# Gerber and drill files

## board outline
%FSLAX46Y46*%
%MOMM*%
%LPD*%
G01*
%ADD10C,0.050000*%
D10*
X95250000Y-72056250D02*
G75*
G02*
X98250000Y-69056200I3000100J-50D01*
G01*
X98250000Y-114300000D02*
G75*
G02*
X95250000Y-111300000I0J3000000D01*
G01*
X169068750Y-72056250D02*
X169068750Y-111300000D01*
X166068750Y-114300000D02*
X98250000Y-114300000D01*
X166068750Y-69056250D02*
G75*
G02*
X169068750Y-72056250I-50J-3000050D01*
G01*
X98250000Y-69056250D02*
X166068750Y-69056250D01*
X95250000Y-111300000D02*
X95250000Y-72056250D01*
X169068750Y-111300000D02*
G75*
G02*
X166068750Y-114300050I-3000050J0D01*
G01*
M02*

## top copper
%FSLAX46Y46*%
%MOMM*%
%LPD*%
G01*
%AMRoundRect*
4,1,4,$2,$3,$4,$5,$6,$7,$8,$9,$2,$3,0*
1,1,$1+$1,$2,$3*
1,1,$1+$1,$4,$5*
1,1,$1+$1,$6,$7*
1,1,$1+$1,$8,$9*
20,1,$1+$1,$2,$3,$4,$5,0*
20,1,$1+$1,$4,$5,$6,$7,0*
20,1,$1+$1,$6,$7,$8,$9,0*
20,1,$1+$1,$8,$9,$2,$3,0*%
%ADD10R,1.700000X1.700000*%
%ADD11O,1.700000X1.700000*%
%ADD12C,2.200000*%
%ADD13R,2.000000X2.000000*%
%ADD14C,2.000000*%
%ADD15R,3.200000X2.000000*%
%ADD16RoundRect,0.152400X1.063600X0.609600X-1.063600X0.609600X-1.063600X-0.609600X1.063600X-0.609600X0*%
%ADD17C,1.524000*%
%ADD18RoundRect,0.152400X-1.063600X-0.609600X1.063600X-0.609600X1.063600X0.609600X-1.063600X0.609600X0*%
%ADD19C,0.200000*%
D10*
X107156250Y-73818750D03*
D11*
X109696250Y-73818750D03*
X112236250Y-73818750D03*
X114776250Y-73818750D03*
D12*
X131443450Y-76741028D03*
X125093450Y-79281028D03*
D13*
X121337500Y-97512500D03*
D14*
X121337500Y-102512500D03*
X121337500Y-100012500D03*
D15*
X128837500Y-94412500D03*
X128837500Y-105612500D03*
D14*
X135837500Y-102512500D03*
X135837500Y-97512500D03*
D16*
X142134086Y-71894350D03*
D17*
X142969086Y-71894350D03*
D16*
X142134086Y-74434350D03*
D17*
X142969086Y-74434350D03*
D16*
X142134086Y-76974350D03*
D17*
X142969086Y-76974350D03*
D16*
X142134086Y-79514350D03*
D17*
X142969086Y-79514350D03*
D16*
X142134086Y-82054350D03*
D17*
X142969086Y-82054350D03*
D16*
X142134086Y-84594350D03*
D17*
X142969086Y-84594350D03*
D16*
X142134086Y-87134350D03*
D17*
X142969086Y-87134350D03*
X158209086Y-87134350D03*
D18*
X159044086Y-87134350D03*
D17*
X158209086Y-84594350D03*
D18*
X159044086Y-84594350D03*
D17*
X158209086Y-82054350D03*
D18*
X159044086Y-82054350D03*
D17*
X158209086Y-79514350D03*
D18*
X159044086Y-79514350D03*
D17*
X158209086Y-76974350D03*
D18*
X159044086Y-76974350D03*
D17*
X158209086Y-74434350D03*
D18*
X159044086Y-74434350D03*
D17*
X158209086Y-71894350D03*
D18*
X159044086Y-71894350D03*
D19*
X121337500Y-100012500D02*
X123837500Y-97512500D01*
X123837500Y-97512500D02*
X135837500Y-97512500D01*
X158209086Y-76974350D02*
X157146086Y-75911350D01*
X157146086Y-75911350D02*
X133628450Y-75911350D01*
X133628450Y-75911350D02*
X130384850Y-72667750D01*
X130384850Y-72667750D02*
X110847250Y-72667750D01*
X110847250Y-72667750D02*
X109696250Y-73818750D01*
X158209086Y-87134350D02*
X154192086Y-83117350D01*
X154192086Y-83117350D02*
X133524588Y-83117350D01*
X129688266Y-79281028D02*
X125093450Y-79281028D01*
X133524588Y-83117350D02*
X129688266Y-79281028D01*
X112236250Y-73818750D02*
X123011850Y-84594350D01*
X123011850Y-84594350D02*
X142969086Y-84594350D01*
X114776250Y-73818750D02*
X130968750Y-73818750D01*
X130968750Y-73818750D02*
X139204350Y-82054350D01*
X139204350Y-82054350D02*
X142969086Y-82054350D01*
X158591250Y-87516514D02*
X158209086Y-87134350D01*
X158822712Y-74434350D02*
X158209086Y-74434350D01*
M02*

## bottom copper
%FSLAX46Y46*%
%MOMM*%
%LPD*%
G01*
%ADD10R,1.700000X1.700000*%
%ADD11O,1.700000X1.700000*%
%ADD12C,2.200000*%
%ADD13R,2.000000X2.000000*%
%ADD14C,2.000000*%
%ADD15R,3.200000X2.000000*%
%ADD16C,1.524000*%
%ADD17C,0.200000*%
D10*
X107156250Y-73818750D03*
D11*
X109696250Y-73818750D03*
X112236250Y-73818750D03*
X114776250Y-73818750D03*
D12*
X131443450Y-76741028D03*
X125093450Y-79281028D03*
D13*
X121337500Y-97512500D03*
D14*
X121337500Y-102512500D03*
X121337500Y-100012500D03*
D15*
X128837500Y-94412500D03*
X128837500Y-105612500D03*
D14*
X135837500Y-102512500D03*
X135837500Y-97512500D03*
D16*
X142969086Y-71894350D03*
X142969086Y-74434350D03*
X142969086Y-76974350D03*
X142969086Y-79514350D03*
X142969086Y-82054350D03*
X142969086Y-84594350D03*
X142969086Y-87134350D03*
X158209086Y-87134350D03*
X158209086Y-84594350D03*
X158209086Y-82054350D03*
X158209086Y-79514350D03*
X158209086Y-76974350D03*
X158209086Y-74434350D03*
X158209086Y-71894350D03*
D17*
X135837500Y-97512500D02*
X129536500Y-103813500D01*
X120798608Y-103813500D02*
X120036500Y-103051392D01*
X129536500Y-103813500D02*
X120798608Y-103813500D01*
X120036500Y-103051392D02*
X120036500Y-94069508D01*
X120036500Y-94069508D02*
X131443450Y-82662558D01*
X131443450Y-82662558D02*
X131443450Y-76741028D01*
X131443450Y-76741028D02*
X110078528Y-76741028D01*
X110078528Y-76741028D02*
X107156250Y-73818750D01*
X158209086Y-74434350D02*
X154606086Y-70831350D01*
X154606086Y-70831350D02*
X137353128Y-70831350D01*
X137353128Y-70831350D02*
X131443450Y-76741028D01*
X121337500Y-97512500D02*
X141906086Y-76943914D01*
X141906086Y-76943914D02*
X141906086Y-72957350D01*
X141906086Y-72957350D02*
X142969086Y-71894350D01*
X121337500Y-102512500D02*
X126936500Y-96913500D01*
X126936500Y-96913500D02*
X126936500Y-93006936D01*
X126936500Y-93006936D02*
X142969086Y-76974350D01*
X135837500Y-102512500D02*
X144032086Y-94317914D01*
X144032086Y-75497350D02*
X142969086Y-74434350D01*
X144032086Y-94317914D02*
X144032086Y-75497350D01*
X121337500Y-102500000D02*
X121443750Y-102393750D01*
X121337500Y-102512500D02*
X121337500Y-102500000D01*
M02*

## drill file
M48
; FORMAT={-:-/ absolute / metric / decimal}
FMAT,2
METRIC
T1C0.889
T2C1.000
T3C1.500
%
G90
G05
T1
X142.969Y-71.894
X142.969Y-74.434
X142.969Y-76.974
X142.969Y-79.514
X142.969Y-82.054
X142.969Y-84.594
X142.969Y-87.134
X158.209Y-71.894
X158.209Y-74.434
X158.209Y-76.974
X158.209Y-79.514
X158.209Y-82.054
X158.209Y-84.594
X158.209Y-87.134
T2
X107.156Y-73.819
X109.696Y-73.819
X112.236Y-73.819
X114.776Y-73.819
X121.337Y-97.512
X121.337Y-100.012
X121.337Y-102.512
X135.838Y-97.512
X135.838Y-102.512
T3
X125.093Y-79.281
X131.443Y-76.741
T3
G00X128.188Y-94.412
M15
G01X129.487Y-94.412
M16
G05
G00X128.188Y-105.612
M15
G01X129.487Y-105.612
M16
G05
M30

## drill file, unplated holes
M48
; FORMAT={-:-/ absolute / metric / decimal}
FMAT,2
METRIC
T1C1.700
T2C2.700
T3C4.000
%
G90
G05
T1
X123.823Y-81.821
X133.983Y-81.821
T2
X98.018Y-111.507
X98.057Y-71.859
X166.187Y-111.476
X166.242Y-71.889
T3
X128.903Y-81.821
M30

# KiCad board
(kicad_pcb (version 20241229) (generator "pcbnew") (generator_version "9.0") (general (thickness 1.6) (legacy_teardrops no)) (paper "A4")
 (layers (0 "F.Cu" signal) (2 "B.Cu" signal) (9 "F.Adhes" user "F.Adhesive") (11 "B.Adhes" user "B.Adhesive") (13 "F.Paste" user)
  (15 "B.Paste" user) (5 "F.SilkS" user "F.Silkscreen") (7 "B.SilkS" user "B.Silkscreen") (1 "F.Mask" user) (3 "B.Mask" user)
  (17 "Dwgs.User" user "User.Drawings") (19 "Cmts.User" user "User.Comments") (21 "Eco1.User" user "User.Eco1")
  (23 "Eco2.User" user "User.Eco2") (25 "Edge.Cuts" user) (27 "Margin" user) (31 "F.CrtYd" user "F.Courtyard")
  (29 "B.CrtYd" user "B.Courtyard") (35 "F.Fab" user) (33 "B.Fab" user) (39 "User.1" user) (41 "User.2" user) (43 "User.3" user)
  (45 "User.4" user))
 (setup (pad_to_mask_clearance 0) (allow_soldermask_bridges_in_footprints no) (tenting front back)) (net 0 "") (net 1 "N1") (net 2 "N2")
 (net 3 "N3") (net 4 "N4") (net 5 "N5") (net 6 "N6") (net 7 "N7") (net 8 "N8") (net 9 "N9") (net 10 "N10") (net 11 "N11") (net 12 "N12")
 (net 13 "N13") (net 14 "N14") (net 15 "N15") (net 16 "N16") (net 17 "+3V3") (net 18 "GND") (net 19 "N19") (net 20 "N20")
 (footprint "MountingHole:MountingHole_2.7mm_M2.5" (layer "F.Cu") (at 166.241551 71.889468)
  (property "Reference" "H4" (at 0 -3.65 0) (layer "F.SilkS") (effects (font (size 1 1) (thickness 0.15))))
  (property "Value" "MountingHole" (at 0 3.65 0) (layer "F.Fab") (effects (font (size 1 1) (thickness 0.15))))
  (pad "" np_thru_hole circle (at 0 0) (size 2.7 2.7) (drill 2.7) (layers "*.Cu" "*.Mask")))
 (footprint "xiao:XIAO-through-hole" (layer "F.Cu") (at 150.589086 79.51435)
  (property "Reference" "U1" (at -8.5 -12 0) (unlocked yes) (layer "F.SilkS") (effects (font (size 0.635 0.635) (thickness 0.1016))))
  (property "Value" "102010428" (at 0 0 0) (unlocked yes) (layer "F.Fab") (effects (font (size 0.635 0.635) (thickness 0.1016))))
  (pad "1" smd roundrect (at -8.455 -7.62 180) (size 2.432 1.524) (layers "F.Cu" "F.Mask") (roundrect_rratio 0.1) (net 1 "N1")
   (thermal_bridge_angle 45))
  (pad "1" thru_hole circle (at -7.62 -7.62 180) (size 1.524 1.524) (drill 0.889) (layers "*.Cu" "*.Mask") (remove_unused_layers no)
   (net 1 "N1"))
  (pad "2" smd roundrect (at -8.455 -5.08 180) (size 2.432 1.524) (layers "F.Cu" "F.Mask") (roundrect_rratio 0.1) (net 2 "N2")
   (thermal_bridge_angle 45))
  (pad "2" thru_hole circle (at -7.62 -5.08 180) (size 1.524 1.524) (drill 0.889) (layers "*.Cu" "*.Mask") (remove_unused_layers no)
   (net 2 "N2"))
  (pad "3" smd roundrect (at -8.455 -2.54 180) (size 2.432 1.524) (layers "F.Cu" "F.Mask") (roundrect_rratio 0.1) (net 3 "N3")
   (thermal_bridge_angle 45))
  (pad "3" thru_hole circle (at -7.62 -2.54 180) (size 1.524 1.524) (drill 0.889) (layers "*.Cu" "*.Mask") (remove_unused_layers no)
   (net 3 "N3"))
  (pad "4" smd roundrect (at -8.455 0 180) (size 2.432 1.524) (layers "F.Cu" "F.Mask") (roundrect_rratio 0.1) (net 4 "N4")
   (thermal_bridge_angle 45))
  (pad "4" thru_hole circle (at -7.62 0 180) (size 1.524 1.524) (drill 0.889) (layers "*.Cu" "*.Mask") (remove_unused_layers no)
   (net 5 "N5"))
  (pad "5" smd roundrect (at -8.455 2.54 180) (size 2.432 1.524) (layers "F.Cu" "F.Mask") (roundrect_rratio 0.1) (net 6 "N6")
   (thermal_bridge_angle 45))
  (pad "5" thru_hole circle (at -7.62 2.54 180) (size 1.524 1.524) (drill 0.889) (layers "*.Cu" "*.Mask") (remove_unused_layers no)
   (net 6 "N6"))
  (pad "6" smd roundrect (at -8.455 5.08 180) (size 2.432 1.524) (layers "F.Cu" "F.Mask") (roundrect_rratio 0.1) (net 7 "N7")
   (thermal_bridge_angle 45))
  (pad "6" thru_hole circle (at -7.62 5.08 180) (size 1.524 1.524) (drill 0.889) (layers "*.Cu" "*.Mask") (remove_unused_layers no)
   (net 7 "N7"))
  (pad "7" smd roundrect (at -8.455 7.62 180) (size 2.432 1.524) (layers "F.Cu" "F.Mask") (roundrect_rratio 0.1) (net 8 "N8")
   (thermal_bridge_angle 45))
  (pad "7" thru_hole circle (at -7.62 7.62 180) (size 1.524 1.524) (drill 0.889) (layers "*.Cu" "*.Mask") (remove_unused_layers no)
   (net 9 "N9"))
  (pad "8" thru_hole circle (at 7.62 7.62) (size 1.524 1.524) (drill 0.889) (layers "*.Cu" "*.Mask") (remove_unused_layers no)
   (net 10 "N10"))
  (pad "8" smd roundrect (at 8.455 7.62) (size 2.432 1.524) (layers "F.Cu" "F.Mask") (roundrect_rratio 0.1) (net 10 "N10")
   (thermal_bridge_angle 45))
  (pad "9" thru_hole circle (at 7.62 5.08) (size 1.524 1.524) (drill 0.889) (layers "*.Cu" "*.Mask") (remove_unused_layers no)
   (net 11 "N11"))
  (pad "9" smd roundrect (at 8.455 5.08) (size 2.432 1.524) (layers "F.Cu" "F.Mask") (roundrect_rratio 0.1) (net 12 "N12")
   (thermal_bridge_angle 45))
  (pad "10" thru_hole circle (at 7.62 2.54) (size 1.524 1.524) (drill 0.889) (layers "*.Cu" "*.Mask") (remove_unused_layers no)
   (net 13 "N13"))
  (pad "10" smd roundrect (at 8.455 2.54) (size 2.432 1.524) (layers "F.Cu" "F.Mask") (roundrect_rratio 0.1) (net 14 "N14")
   (thermal_bridge_angle 45))
  (pad "11" thru_hole circle (at 7.62 0) (size 1.524 1.524) (drill 0.889) (layers "*.Cu" "*.Mask") (remove_unused_layers no) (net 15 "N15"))
  (pad "11" smd roundrect (at 8.455 0) (size 2.432 1.524) (layers "F.Cu" "F.Mask") (roundrect_rratio 0.1) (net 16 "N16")
   (thermal_bridge_angle 45))
  (pad "12" thru_hole circle (at 7.62 -2.54) (size 1.524 1.524) (drill 0.889) (layers "*.Cu" "*.Mask") (remove_unused_layers no)
   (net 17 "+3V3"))
  (pad "12" smd roundrect (at 8.455 -2.54) (size 2.432 1.524) (layers "F.Cu" "F.Mask") (roundrect_rratio 0.1) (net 17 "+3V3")
   (thermal_bridge_angle 45))
  (pad "13" thru_hole circle (at 7.62 -5.08) (size 1.524 1.524) (drill 0.889) (layers "*.Cu" "*.Mask") (remove_unused_layers no)
   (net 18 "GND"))
  (pad "13" smd roundrect (at 8.455 -5.08) (size 2.432 1.524) (layers "F.Cu" "F.Mask") (roundrect_rratio 0.1) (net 18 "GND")
   (thermal_bridge_angle 45))
  (pad "14" thru_hole circle (at 7.62 -7.62) (size 1.524 1.524) (drill 0.889) (layers "*.Cu" "*.Mask") (remove_unused_layers no)
   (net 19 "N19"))
  (pad "14" smd roundrect (at 8.455 -7.62) (size 2.432 1.524) (layers "F.Cu" "F.Mask") (roundrect_rratio 0.1) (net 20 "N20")
   (thermal_bridge_angle 45)))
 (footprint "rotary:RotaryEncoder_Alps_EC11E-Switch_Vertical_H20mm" (layer "F.Cu") (at 121.3375 97.5125)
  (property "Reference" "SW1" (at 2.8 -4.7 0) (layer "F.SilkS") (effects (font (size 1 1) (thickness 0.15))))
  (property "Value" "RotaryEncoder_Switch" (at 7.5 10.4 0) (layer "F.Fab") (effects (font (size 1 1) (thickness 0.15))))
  (pad "A" thru_hole rect (at 0 0) (size 2 2) (drill 1) (layers "*.Cu" "*.Mask") (remove_unused_layers no) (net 1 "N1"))
  (pad "B" thru_hole circle (at 0 5) (size 2 2) (drill 1) (layers "*.Cu" "*.Mask") (remove_unused_layers no) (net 3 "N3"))
  (pad "C" thru_hole circle (at 0 2.5) (size 2 2) (drill 1) (layers "*.Cu" "*.Mask") (remove_unused_layers no) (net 18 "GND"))
  (pad "MP" thru_hole rect (at 7.5 -3.1) (size 3.2 2) (drill oval 2.8 1.5) (layers "*.Cu" "*.Mask") (remove_unused_layers no))
  (pad "MP" thru_hole rect (at 7.5 8.1) (size 3.2 2) (drill oval 2.8 1.5) (layers "*.Cu" "*.Mask") (remove_unused_layers no))
  (pad "S1" thru_hole circle (at 14.5 5) (size 2 2) (drill 1) (layers "*.Cu" "*.Mask") (remove_unused_layers no) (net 2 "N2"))
  (pad "S2" thru_hole circle (at 14.5 0) (size 2 2) (drill 1) (layers "*.Cu" "*.Mask") (remove_unused_layers no) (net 18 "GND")))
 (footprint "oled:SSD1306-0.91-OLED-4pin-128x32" (layer "F.Cu") (at 104.96625 110.31875 90)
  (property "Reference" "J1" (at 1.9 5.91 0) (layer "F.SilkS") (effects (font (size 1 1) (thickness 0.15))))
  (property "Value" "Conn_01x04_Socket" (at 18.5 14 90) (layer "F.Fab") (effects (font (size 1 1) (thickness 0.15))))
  (pad "1" thru_hole rect (at 36.5 2.19 90) (size 1.7 1.7) (drill 1) (layers "*.Cu" "*.Mask") (remove_unused_layers no) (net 18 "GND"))
  (pad "2" thru_hole oval (at 36.5 4.73 90) (size 1.7 1.7) (drill 1) (layers "*.Cu" "*.Mask") (remove_unused_layers no) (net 17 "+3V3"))
  (pad "3" thru_hole oval (at 36.5 7.27 90) (size 1.7 1.7) (drill 1) (layers "*.Cu" "*.Mask") (remove_unused_layers no) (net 7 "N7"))
  (pad "4" thru_hole oval (at 36.5 9.81 90) (size 1.7 1.7) (drill 1) (layers "*.Cu" "*.Mask") (remove_unused_layers no) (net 6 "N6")))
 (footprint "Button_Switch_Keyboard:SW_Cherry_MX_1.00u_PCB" (layer "F.Cu") (at 131.44345 76.741028)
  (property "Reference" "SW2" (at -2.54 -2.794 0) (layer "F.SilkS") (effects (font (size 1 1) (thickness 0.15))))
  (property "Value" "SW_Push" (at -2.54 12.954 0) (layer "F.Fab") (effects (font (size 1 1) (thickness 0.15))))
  (pad "" np_thru_hole circle (at -7.62 5.08) (size 1.7 1.7) (drill 1.7) (layers "*.Cu" "*.Mask"))
  (pad "" np_thru_hole circle (at -2.54 5.08) (size 4 4) (drill 4) (layers "*.Cu" "*.Mask"))
  (pad "" np_thru_hole circle (at 2.54 5.08) (size 1.7 1.7) (drill 1.7) (layers "*.Cu" "*.Mask"))
  (pad "1" thru_hole circle (at 0 0) (size 2.2 2.2) (drill 1.5) (layers "*.Cu" "*.Mask") (remove_unused_layers no) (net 18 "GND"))
  (pad "2" thru_hole circle (at -6.35 2.54) (size 2.2 2.2) (drill 1.5) (layers "*.Cu" "*.Mask") (remove_unused_layers no) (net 10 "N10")))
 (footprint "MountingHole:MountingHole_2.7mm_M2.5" (layer "F.Cu") (at 98.056834 71.858552)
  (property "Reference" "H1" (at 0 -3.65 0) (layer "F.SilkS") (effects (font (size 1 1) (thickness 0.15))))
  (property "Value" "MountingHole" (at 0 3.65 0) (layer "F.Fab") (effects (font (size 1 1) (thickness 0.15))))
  (pad "" np_thru_hole circle (at 0 0) (size 2.7 2.7) (drill 2.7) (layers "*.Cu" "*.Mask")))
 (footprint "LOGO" (layer "F.Cu") (at 147.6375 100.0125)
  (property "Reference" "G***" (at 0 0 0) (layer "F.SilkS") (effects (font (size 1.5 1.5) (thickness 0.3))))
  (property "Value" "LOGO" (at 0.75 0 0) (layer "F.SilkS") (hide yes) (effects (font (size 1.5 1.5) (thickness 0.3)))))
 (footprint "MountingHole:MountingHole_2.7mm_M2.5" (layer "F.Cu") (at 166.186859 111.475774)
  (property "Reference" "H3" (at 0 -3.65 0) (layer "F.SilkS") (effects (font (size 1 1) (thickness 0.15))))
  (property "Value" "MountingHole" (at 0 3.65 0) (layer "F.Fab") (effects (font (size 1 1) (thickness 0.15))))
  (pad "" np_thru_hole circle (at 0 0) (size 2.7 2.7) (drill 2.7) (layers "*.Cu" "*.Mask")))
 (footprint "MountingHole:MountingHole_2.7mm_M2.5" (layer "F.Cu") (at 98.017649 111.507208)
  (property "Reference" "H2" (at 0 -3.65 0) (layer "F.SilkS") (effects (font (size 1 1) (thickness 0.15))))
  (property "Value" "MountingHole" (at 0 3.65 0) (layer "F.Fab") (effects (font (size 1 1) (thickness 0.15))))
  (pad "" np_thru_hole circle (at 0 0) (size 2.7 2.7) (drill 2.7) (layers "*.Cu" "*.Mask")))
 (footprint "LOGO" (layer "B.Cu") (at 130.96875 90.4875 180)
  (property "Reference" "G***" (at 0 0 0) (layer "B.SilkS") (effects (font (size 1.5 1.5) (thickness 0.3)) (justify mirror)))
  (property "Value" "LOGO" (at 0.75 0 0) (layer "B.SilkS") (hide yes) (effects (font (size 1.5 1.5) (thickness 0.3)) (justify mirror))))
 (gr_arc (start 95.25 72.05625) (mid 96.128697 69.934962) (end 98.25 69.05625) (stroke (width 0.05) (type default)) (layer "Edge.Cuts"))
 (gr_arc (start 98.25 114.3) (mid 96.12868 113.42132) (end 95.25 111.3) (stroke (width 0.05) (type default)) (layer "Edge.Cuts"))
 (gr_line (start 169.06875 72.05625) (end 169.06875 111.3) (stroke (width 0.05) (type default)) (layer "Edge.Cuts"))
 (gr_line (start 166.06875 114.3) (end 98.25 114.3) (stroke (width 0.05) (type default)) (layer "Edge.Cuts"))
 (gr_arc (start 166.06875 69.05625) (mid 168.19007 69.93493) (end 169.06875 72.05625) (stroke (width 0.05) (type default))
  (layer "Edge.Cuts"))
 (gr_line (start 98.25 69.05625) (end 166.06875 69.05625) (stroke (width 0.05) (type default)) (layer "Edge.Cuts"))
 (gr_line (start 95.25 111.3) (end 95.25 72.05625) (stroke (width 0.05) (type default)) (layer "Edge.Cuts"))
 (gr_arc (start 169.06875 111.3) (mid 168.19007 113.42132) (end 166.06875 114.3) (stroke (width 0.05) (type default)) (layer "Edge.Cuts"))
 (segment (start 158.209086 76.97435) (end 157.146086 75.91135) (width 0.2) (layer "F.Cu") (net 17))
 (segment (start 157.146086 75.91135) (end 133.62845 75.91135) (width 0.2) (layer "F.Cu") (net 17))
 (segment (start 110.84725 72.66775) (end 109.69625 73.81875) (width 0.2) (layer "F.Cu") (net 17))
 (segment (start 130.38485 72.66775) (end 110.84725 72.66775) (width 0.2) (layer "F.Cu") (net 17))
 (segment (start 133.62845 75.91135) (end 130.38485 72.66775) (width 0.2) (layer "F.Cu") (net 17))
 (segment (start 114.77625 73.81875) (end 130.96875 73.81875) (width 0.2) (layer "F.Cu") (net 6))
 (segment (start 139.20435 82.05435) (end 142.969086 82.05435) (width 0.2) (layer "F.Cu") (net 6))
 (segment (start 130.96875 73.81875) (end 139.20435 82.05435) (width 0.2) (layer "F.Cu") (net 6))
 (segment (start 123.8375 97.5125) (end 135.8375 97.5125) (width 0.2) (layer "F.Cu") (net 18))
 (segment (start 158.822712 74.43435) (end 158.209086 74.43435) (width 0.2) (layer "F.Cu") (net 18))
 (segment (start 121.3375 100.0125) (end 123.8375 97.5125) (width 0.2) (layer "F.Cu") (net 18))
 (segment (start 154.606086 70.83135) (end 137.353128 70.83135) (width 0.2) (layer "B.Cu") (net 18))
 (segment (start 120.0365 94.069508) (end 131.44345 82.662558) (width 0.2) (layer "B.Cu") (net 18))
 (segment (start 137.353128 70.83135) (end 131.44345 76.741028) (width 0.2) (layer "B.Cu") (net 18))
 (segment (start 131.44345 82.662558) (end 131.44345 76.741028) (width 0.2) (layer "B.Cu") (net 18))
 (segment (start 135.8375 97.5125) (end 129.5365 103.8135) (width 0.2) (layer "B.Cu") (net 18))
 (segment (start 120.798608 103.8135) (end 120.0365 103.051392) (width 0.2) (layer "B.Cu") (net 18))
 (segment (start 129.5365 103.8135) (end 120.798608 103.8135) (width 0.2) (layer "B.Cu") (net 18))
 (segment (start 131.44345 76.741028) (end 110.078528 76.741028) (width 0.2) (layer "B.Cu") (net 18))
 (segment (start 120.0365 103.051392) (end 120.0365 94.069508) (width 0.2) (layer "B.Cu") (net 18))
 (segment (start 110.078528 76.741028) (end 107.15625 73.81875) (width 0.2) (layer "B.Cu") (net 18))
 (segment (start 158.209086 74.43435) (end 154.606086 70.83135) (width 0.2) (layer "B.Cu") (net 18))
 (segment (start 112.23625 73.81875) (end 123.01185 84.59435) (width 0.2) (layer "F.Cu") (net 7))
 (segment (start 123.01185 84.59435) (end 142.969086 84.59435) (width 0.2) (layer "F.Cu") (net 7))
 (segment (start 126.9365 93.006936) (end 142.969086 76.97435) (width 0.2) (layer "B.Cu") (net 3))
 (segment (start 121.3375 102.5) (end 121.44375 102.39375) (width 0.2) (layer "B.Cu") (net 3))
 (segment (start 121.3375 102.5125) (end 121.3375 102.5) (width 0.2) (layer "B.Cu") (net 3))
 (segment (start 126.9365 96.9135) (end 126.9365 93.006936) (width 0.2) (layer "B.Cu") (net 3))
 (segment (start 121.3375 102.5125) (end 126.9365 96.9135) (width 0.2) (layer "B.Cu") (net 3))
 (segment (start 141.906086 76.943914) (end 141.906086 72.95735) (width 0.2) (layer "B.Cu") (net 1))
 (segment (start 121.3375 97.5125) (end 141.906086 76.943914) (width 0.2) (layer "B.Cu") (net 1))
 (segment (start 141.906086 72.95735) (end 142.969086 71.89435) (width 0.2) (layer "B.Cu") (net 1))
 (segment (start 144.032086 75.49735) (end 142.969086 74.43435) (width 0.2) (layer "B.Cu") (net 2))
 (segment (start 144.032086 94.317914) (end 144.032086 75.49735) (width 0.2) (layer "B.Cu") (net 2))
 (segment (start 135.8375 102.5125) (end 144.032086 94.317914) (width 0.2) (layer "B.Cu") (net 2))
 (segment (start 154.192086 83.11735) (end 133.524588 83.11735) (width 0.2) (layer "F.Cu") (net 10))
 (segment (start 158.59125 87.516514) (end 158.209086 87.13435) (width 0.2) (layer "F.Cu") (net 10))
 (segment (start 133.524588 83.11735) (end 129.688266 79.281028) (width 0.2) (layer "F.Cu") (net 10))
 (segment (start 129.688266 79.281028) (end 125.09345 79.281028) (width 0.2) (layer "F.Cu") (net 10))
 (segment (start 158.209086 87.13435) (end 154.192086 83.11735) (width 0.2) (layer "F.Cu") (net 10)))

